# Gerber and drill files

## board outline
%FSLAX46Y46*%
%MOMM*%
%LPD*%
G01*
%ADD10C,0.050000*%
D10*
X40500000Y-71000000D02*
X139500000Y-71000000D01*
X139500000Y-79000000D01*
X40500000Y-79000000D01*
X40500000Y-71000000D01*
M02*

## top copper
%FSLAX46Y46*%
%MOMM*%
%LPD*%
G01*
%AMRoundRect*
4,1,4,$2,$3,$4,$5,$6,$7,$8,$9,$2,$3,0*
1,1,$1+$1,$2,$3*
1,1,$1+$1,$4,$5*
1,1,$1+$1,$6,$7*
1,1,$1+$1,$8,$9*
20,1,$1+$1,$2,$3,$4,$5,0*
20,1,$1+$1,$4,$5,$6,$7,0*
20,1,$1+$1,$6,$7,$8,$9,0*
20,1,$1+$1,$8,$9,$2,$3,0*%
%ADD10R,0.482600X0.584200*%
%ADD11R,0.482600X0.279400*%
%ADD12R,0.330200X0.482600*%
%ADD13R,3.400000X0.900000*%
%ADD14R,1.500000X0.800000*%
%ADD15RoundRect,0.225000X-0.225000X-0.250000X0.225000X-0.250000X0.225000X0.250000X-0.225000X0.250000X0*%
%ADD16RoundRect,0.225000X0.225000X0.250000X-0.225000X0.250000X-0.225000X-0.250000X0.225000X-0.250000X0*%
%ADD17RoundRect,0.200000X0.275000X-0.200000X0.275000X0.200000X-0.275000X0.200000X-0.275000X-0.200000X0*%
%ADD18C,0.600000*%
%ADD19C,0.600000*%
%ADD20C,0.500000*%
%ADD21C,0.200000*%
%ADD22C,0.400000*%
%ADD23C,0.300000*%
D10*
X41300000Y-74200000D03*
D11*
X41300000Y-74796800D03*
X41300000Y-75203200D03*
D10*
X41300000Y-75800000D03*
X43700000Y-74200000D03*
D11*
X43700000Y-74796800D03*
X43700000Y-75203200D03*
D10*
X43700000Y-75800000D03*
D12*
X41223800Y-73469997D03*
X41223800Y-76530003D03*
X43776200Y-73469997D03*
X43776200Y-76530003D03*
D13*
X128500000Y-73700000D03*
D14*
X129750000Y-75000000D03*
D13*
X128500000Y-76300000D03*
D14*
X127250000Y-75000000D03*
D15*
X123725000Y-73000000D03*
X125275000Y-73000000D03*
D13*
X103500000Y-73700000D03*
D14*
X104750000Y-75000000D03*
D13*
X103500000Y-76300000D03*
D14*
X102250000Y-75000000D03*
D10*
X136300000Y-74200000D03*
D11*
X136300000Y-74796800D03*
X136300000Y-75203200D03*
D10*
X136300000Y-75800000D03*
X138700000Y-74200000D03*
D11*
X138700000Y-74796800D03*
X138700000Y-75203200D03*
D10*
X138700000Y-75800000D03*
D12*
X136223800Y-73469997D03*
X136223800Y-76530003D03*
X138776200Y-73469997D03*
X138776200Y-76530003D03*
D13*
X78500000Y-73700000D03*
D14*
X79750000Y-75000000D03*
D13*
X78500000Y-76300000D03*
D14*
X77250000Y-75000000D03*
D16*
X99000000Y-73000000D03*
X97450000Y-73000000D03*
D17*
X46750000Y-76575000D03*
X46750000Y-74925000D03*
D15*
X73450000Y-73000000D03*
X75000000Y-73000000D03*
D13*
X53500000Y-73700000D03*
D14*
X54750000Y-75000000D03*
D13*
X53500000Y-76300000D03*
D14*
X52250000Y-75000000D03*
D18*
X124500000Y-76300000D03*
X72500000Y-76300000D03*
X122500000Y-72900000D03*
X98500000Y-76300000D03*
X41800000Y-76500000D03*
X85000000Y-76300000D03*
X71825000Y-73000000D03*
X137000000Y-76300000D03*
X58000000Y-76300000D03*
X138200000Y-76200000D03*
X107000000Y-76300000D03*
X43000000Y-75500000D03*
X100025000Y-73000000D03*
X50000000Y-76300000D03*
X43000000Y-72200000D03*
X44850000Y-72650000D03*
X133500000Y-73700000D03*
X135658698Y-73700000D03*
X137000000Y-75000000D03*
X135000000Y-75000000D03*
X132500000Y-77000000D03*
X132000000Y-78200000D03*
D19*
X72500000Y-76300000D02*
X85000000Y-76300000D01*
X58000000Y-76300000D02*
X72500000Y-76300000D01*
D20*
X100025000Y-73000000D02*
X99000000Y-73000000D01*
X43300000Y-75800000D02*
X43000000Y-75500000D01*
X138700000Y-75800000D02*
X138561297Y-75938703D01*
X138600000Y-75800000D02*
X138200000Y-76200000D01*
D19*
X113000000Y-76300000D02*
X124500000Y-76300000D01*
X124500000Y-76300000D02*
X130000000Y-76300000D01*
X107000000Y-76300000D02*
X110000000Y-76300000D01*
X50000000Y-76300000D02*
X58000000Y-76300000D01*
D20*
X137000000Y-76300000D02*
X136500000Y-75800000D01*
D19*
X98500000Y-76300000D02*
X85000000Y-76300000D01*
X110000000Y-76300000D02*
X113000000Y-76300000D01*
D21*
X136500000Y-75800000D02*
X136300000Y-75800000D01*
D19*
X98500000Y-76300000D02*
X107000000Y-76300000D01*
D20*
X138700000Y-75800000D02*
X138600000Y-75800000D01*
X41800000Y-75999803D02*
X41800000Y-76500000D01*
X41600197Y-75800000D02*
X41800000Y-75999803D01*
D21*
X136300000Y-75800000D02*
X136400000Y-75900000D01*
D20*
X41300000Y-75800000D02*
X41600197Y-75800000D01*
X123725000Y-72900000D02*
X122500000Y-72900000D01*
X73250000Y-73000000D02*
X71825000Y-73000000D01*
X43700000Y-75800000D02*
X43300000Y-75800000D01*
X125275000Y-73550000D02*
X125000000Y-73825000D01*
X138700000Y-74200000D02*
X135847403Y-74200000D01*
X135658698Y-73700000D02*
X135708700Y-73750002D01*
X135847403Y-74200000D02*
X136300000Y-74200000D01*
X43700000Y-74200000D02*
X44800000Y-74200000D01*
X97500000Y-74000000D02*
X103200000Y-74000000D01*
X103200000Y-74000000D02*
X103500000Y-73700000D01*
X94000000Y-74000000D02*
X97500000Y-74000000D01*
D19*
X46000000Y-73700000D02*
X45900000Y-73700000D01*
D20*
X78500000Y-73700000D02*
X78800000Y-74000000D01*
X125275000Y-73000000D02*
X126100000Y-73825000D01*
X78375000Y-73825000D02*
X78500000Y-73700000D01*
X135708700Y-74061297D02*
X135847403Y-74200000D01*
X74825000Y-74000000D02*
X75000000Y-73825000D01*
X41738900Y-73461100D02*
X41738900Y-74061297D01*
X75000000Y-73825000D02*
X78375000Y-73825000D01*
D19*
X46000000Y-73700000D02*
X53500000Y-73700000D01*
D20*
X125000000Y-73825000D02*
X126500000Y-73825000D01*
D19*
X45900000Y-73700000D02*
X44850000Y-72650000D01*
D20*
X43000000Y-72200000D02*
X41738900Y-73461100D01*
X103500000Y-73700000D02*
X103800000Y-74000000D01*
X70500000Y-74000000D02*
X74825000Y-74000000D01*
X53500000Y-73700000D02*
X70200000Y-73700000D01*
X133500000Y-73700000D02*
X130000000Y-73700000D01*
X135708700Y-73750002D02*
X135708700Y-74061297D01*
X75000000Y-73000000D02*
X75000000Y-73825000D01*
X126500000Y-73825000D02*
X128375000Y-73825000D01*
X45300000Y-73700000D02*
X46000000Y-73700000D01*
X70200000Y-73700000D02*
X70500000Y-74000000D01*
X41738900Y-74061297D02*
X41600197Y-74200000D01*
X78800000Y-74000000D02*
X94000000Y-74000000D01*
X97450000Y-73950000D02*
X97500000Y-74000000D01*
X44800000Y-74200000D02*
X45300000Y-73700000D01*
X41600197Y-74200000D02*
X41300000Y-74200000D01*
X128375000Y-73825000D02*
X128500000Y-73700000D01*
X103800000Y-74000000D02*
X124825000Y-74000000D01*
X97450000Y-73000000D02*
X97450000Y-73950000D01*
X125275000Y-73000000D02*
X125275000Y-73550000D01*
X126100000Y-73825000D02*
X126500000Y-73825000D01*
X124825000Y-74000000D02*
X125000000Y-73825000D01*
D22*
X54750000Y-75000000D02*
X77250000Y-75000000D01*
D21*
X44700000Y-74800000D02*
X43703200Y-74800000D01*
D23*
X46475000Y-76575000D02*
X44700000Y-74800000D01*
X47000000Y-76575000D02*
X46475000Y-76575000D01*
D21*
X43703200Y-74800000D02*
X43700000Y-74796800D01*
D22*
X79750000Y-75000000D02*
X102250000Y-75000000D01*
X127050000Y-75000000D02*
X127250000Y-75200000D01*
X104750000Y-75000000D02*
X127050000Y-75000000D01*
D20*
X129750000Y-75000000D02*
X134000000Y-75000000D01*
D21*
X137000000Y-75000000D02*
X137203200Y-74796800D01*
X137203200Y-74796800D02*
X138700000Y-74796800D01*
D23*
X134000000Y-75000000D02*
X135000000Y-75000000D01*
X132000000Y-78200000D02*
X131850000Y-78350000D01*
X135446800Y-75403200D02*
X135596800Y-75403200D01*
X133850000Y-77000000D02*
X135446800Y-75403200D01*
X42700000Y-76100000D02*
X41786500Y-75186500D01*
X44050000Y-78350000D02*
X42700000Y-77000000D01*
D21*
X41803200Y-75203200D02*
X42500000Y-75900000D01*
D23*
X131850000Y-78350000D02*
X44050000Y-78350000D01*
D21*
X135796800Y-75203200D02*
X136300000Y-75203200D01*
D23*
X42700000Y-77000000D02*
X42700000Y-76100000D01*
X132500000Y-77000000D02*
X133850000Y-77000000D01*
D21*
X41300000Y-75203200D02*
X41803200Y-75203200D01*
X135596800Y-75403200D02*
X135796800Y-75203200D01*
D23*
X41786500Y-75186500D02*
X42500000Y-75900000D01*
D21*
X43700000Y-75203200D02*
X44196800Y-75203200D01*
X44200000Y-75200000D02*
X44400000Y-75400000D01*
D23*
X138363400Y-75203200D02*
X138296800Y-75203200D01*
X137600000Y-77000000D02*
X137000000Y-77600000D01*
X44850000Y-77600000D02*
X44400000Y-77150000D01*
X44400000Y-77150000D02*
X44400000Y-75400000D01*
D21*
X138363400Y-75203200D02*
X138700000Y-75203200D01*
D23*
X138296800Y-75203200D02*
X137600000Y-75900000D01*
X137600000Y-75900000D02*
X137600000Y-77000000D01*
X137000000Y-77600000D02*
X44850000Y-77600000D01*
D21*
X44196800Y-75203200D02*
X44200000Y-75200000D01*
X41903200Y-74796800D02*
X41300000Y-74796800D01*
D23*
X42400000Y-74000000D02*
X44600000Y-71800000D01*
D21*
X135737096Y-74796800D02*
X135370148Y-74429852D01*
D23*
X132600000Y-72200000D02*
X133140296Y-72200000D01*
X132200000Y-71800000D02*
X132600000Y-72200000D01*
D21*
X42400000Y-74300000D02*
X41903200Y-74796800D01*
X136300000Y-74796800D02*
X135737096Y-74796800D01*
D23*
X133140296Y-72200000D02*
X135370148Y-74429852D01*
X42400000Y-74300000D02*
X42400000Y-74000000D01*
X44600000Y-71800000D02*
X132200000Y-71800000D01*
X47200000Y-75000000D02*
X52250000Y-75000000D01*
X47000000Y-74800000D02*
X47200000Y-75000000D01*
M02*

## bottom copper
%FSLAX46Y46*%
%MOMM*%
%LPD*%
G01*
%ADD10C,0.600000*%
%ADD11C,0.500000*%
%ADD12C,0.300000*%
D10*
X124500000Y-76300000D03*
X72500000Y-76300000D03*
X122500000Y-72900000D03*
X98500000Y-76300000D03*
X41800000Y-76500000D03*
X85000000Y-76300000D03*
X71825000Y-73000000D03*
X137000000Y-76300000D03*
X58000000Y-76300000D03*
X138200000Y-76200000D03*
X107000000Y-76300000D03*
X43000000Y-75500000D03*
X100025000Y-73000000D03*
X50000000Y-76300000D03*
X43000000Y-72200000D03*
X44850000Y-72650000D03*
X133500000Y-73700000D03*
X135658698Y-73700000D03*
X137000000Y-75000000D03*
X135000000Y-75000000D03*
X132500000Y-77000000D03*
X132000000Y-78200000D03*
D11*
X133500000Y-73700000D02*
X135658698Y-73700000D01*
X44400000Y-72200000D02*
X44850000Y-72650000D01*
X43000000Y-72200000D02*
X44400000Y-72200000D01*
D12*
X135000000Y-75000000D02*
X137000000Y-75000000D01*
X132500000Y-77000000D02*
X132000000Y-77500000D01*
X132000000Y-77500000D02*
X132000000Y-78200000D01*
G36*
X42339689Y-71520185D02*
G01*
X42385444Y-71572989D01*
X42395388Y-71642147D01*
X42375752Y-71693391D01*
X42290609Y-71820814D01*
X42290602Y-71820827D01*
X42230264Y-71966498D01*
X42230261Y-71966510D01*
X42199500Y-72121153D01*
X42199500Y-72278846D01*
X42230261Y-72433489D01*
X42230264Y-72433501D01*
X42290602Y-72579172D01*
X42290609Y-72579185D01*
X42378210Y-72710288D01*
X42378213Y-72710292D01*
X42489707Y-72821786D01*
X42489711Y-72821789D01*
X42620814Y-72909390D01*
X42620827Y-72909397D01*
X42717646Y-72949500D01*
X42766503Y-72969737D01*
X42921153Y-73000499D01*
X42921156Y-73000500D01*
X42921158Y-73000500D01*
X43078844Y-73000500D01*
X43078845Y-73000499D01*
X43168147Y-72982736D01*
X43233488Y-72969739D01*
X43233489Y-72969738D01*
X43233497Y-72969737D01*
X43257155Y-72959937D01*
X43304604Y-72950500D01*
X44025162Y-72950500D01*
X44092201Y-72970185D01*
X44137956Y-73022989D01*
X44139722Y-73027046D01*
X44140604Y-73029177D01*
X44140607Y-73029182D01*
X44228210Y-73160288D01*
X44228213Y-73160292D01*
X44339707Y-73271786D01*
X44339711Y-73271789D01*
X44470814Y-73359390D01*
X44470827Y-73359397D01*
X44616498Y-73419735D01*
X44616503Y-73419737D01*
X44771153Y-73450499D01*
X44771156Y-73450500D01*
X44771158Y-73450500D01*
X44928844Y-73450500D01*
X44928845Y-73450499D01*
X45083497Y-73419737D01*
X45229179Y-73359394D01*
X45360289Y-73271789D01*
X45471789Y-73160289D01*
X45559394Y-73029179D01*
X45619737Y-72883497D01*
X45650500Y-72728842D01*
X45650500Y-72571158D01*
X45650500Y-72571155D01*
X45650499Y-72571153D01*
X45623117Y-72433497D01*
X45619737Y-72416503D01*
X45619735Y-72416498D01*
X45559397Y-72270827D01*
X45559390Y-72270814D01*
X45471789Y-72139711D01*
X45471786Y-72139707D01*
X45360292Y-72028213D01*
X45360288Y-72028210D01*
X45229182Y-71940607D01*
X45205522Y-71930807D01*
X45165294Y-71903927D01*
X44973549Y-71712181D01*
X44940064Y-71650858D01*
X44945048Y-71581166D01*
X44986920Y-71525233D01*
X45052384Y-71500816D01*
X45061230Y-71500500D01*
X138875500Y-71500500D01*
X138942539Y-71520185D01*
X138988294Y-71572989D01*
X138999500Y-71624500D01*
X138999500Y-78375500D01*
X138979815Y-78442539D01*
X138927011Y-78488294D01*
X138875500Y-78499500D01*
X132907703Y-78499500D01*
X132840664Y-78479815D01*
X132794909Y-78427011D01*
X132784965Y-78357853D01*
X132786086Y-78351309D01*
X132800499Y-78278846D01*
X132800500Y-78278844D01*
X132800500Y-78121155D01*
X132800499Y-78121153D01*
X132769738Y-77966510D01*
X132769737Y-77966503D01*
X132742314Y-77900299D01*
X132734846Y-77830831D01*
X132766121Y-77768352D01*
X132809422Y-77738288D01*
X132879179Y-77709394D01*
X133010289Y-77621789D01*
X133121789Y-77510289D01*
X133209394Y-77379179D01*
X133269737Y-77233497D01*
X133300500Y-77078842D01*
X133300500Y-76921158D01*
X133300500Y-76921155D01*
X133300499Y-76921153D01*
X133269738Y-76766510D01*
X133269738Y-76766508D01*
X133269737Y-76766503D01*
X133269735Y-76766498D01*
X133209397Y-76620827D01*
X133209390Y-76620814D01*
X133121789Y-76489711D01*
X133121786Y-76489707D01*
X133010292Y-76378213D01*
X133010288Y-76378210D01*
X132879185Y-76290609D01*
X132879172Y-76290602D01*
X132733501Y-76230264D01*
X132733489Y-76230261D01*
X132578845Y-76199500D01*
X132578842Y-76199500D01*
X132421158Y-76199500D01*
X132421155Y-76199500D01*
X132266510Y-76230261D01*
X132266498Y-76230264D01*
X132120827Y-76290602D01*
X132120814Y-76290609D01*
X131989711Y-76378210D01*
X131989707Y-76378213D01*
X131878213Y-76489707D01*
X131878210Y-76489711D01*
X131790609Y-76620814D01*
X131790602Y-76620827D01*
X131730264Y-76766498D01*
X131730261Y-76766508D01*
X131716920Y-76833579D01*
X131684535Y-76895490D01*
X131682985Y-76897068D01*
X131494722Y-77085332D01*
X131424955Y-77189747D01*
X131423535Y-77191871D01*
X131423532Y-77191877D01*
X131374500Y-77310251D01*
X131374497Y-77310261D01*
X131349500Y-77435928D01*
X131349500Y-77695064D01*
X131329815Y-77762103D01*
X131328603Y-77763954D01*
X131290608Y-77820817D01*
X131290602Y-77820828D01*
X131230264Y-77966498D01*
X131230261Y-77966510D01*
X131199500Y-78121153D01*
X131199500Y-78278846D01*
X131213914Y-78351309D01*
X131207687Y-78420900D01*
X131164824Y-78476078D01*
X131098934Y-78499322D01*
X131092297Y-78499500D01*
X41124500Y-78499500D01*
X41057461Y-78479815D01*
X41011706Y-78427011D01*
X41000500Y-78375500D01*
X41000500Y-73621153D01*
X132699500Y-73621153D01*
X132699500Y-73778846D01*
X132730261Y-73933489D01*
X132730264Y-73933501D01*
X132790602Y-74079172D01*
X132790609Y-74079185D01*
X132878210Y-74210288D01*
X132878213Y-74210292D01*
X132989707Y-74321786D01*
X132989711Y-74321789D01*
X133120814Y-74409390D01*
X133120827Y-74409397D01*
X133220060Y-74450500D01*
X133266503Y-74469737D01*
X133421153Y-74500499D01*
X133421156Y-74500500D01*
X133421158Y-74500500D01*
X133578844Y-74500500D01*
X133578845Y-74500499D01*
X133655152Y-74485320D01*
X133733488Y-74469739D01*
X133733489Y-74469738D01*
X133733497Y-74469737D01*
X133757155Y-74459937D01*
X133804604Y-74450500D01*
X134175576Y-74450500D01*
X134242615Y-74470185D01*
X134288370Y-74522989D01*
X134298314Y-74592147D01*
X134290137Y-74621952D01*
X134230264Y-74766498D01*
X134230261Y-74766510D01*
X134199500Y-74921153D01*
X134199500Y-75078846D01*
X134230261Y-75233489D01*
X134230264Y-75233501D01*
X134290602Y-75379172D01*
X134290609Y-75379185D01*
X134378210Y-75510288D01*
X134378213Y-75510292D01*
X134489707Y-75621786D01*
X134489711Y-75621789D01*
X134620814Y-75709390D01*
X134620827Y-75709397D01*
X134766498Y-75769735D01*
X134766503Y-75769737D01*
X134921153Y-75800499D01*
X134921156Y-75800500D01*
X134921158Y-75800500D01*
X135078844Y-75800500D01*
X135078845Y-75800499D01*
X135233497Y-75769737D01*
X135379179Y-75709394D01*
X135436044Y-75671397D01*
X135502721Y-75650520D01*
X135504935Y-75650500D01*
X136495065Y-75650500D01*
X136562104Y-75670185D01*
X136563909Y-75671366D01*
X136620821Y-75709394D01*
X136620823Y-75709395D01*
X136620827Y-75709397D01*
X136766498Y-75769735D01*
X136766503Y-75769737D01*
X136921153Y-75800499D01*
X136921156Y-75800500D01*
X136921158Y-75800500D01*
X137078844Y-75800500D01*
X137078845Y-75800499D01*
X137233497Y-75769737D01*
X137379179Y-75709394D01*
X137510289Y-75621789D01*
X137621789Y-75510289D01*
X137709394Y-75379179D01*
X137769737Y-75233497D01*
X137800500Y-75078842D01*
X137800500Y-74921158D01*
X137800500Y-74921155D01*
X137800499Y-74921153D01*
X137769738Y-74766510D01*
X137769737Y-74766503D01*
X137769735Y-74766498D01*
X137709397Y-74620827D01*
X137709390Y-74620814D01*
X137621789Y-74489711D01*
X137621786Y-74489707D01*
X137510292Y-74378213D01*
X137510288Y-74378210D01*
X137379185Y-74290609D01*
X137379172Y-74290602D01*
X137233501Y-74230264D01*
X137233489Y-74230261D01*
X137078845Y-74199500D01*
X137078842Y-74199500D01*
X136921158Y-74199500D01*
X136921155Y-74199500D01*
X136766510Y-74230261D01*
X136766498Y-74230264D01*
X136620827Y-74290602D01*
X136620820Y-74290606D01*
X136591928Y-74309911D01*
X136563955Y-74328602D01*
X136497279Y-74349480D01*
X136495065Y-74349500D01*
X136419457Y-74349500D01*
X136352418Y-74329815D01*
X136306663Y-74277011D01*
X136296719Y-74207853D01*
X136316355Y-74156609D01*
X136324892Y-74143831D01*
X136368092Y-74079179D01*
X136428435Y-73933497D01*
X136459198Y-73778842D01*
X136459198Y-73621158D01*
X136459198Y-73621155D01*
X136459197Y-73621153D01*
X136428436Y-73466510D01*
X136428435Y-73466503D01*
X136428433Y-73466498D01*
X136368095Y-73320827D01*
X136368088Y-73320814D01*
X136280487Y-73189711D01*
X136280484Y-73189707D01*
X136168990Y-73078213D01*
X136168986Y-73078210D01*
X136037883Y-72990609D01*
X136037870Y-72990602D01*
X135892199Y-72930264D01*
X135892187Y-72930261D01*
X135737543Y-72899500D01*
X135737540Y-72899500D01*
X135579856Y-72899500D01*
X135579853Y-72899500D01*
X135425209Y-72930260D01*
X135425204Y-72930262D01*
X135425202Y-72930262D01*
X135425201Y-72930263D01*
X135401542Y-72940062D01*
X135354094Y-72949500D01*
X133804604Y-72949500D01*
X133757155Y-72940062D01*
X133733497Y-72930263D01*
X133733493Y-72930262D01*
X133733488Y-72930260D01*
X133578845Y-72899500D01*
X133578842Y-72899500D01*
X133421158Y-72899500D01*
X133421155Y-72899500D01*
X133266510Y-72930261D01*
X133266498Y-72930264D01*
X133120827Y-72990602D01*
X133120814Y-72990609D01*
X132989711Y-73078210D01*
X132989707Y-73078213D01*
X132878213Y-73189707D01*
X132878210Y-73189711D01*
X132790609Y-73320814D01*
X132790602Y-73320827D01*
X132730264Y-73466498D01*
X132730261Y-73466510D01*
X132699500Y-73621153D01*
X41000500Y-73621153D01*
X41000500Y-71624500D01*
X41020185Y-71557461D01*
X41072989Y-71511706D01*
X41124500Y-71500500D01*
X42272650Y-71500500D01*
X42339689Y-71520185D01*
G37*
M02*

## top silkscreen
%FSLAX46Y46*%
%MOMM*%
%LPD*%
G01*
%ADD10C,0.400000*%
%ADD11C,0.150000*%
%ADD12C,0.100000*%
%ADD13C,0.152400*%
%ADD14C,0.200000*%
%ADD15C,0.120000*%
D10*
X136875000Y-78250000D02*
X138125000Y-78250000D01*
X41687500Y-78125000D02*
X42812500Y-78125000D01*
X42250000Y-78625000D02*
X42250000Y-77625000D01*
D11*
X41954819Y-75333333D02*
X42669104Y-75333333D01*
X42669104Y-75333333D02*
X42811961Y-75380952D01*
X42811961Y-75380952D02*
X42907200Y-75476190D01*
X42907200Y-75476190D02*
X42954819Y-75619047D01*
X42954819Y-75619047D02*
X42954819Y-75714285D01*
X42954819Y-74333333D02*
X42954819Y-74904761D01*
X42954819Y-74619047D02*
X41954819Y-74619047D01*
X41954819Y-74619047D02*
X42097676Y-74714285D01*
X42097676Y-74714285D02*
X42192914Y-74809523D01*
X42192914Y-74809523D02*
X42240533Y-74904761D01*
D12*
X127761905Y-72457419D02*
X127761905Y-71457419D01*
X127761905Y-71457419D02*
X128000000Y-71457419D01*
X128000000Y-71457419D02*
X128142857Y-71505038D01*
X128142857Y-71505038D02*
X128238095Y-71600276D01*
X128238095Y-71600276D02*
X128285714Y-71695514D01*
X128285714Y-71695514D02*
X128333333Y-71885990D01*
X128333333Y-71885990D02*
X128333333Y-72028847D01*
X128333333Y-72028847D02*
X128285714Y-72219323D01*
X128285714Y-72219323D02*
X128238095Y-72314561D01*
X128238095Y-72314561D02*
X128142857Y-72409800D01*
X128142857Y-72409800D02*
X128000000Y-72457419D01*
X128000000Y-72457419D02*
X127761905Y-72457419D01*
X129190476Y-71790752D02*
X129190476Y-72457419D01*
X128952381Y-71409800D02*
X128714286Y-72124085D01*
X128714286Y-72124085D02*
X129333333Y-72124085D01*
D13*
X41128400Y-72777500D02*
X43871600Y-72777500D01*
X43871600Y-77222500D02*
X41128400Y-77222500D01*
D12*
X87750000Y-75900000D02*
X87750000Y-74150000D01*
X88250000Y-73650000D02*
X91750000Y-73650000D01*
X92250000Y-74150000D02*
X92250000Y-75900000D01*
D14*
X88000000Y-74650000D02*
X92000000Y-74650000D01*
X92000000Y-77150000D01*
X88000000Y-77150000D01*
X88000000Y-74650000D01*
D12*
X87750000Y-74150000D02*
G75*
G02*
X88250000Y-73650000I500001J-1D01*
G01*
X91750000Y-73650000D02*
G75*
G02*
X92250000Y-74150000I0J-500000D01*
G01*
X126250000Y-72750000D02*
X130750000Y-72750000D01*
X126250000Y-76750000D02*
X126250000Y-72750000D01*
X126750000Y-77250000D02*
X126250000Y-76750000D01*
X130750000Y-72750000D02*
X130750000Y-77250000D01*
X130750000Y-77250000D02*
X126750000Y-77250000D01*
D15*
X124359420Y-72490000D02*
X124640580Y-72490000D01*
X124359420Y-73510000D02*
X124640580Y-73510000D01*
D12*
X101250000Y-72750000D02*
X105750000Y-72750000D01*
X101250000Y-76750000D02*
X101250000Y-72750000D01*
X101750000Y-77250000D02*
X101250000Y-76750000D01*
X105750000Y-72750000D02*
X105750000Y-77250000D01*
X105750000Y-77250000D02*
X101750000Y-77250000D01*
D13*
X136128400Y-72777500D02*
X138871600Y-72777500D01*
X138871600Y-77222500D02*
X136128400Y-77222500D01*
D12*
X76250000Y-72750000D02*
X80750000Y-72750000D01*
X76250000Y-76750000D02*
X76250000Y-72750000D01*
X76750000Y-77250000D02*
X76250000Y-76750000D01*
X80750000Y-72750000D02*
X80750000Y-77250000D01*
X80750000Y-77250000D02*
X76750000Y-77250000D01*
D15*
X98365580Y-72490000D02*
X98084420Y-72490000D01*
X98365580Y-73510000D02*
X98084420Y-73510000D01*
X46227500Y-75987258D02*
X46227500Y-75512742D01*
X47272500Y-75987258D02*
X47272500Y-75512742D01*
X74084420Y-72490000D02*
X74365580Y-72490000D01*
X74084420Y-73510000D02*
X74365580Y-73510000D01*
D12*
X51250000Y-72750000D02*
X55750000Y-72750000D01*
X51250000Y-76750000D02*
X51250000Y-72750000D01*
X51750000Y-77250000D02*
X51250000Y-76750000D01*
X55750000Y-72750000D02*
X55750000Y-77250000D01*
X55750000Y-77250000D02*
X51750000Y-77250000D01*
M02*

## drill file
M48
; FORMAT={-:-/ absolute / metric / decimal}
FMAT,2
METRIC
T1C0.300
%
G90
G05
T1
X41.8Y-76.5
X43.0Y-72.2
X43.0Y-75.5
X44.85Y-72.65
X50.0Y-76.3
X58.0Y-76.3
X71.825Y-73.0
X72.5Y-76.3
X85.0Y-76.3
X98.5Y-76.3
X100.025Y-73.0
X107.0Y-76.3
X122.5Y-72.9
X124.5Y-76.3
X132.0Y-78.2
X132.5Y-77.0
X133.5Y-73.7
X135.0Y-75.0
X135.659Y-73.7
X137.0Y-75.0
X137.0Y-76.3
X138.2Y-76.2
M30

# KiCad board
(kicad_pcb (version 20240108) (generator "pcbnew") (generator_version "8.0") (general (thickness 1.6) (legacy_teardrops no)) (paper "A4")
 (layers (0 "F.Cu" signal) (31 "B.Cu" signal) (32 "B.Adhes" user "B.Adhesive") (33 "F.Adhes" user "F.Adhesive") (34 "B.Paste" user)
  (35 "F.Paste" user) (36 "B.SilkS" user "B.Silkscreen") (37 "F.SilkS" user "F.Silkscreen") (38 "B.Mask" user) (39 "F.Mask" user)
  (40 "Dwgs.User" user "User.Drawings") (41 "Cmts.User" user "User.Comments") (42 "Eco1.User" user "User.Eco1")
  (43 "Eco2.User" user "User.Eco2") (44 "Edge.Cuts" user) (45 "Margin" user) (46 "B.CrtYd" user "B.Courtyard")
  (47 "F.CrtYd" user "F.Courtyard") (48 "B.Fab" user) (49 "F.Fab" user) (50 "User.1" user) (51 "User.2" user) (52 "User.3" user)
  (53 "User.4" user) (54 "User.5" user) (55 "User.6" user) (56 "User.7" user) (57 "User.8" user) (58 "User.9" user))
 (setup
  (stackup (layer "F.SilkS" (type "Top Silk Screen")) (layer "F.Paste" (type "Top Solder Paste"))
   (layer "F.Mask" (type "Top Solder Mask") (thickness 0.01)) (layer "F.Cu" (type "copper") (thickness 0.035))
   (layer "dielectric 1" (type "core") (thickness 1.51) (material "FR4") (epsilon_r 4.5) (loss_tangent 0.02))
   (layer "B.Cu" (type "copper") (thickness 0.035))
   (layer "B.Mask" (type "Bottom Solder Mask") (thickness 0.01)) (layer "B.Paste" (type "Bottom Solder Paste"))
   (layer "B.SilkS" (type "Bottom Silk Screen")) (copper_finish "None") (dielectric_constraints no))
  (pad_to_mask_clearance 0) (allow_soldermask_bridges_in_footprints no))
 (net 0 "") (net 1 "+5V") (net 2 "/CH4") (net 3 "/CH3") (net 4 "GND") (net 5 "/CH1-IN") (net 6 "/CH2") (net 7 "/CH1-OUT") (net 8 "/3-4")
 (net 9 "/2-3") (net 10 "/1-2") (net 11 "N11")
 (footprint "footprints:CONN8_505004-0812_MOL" (layer "F.Cu") (at 42.5 75 90)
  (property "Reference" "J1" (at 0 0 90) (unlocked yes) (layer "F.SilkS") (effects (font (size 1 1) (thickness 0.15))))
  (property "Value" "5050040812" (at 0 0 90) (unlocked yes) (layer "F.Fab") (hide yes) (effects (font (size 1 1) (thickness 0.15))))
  (fp_line (start 2.2225 -1.3716) (end 2.2225 1.3716) (stroke (width 0.1524) (type solid)) (layer "F.SilkS"))
  (fp_line (start -2.2225 1.3716) (end -2.2225 -1.3716) (stroke (width 0.1524) (type solid)) (layer "F.SilkS"))
  (pad "1" smd rect (at 0.8 -1.2 90) (size 0.5842 0.4826) (layers "F.Cu" "F.Paste" "F.Mask") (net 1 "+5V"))
  (pad "2" smd rect (at 0.2032 -1.2 90) (size 0.2794 0.4826) (layers "F.Cu" "F.Paste" "F.Mask") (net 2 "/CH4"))
  (pad "3" smd rect (at -0.2032 -1.2 90) (size 0.2794 0.4826) (layers "F.Cu" "F.Paste" "F.Mask") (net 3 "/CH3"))
  (pad "4" smd rect (at -0.8 -1.2 90) (size 0.5842 0.4826) (layers "F.Cu" "F.Paste" "F.Mask") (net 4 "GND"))
  (pad "5" smd rect (at 0.8 1.2 90) (size 0.5842 0.4826) (layers "F.Cu" "F.Paste" "F.Mask") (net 1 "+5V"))
  (pad "6" smd rect (at 0.2032 1.2 90) (size 0.2794 0.4826) (layers "F.Cu" "F.Paste" "F.Mask") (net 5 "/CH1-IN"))
  (pad "7" smd rect (at -0.2032 1.2 90) (size 0.2794 0.4826) (layers "F.Cu" "F.Paste" "F.Mask") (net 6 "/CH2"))
  (pad "8" smd rect (at -0.8 1.2 90) (size 0.5842 0.4826) (layers "F.Cu" "F.Paste" "F.Mask") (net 4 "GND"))
  (pad "9" smd rect (at 1.530003 -1.2762 90) (size 0.4826 0.3302) (layers "F.Cu" "F.Paste" "F.Mask"))
  (pad "10" smd rect (at -1.530003 -1.2762 90) (size 0.4826 0.3302) (layers "F.Cu" "F.Paste" "F.Mask"))
  (pad "11" smd rect (at 1.530003 1.2762 90) (size 0.4826 0.3302) (layers "F.Cu" "F.Paste" "F.Mask"))
  (pad "12" smd rect (at -1.530003 1.2762 90) (size 0.4826 0.3302) (layers "F.Cu" "F.Paste" "F.Mask")))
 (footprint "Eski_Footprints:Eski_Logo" (layer "F.Cu") (at 90 77.15)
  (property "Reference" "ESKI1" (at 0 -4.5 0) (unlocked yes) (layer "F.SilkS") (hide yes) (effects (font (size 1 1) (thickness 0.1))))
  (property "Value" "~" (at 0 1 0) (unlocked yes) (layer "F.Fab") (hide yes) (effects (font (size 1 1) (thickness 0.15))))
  (fp_line (start -2.25 -1.25) (end -2.25 -3) (stroke (width 0.1) (type default)) (layer "F.SilkS"))
  (fp_line (start -1.75 -3.5) (end 1.75 -3.5) (stroke (width 0.1) (type default)) (layer "F.SilkS"))
  (fp_line (start 2.25 -3) (end 2.25 -1.25) (stroke (width 0.1) (type default)) (layer "F.SilkS"))
  (fp_rect (start -2 -2.5) (end 2 0) (stroke (width 0.2) (type default)) (fill none) (layer "F.SilkS"))
  (fp_arc (start -2.25 -3) (mid -2.103553 -3.353553) (end -1.75 -3.5) (stroke (width 0.1) (type default)) (layer "F.SilkS"))
  (fp_arc (start 1.75 -3.5) (mid 2.103553 -3.353553) (end 2.25 -3) (stroke (width 0.1) (type default)) (layer "F.SilkS")))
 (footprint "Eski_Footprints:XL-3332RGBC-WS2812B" (layer "F.Cu") (at 128.5 75)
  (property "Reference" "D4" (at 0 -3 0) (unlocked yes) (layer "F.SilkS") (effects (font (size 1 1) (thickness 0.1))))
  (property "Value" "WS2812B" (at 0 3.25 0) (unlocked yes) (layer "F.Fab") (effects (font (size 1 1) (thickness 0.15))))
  (fp_line (start -2.25 -2.25) (end 2.25 -2.25) (stroke (width 0.1) (type default)) (layer "F.SilkS"))
  (fp_line (start -2.25 1.75) (end -2.25 -2.25) (stroke (width 0.1) (type default)) (layer "F.SilkS"))
  (fp_line (start -1.75 2.25) (end -2.25 1.75) (stroke (width 0.1) (type default)) (layer "F.SilkS"))
  (fp_line (start 2.25 -2.25) (end 2.25 2.25) (stroke (width 0.1) (type default)) (layer "F.SilkS"))
  (fp_line (start 2.25 2.25) (end -1.75 2.25) (stroke (width 0.1) (type default)) (layer "F.SilkS"))
  (pad "1" smd rect (at 0 -1.3) (size 3.4 0.9) (layers "F.Cu" "F.Paste" "F.Mask") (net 1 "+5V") (thermal_bridge_angle 45))
  (pad "2" smd rect (at 1.25 0) (size 1.5 0.8) (layers "F.Cu" "F.Paste" "F.Mask") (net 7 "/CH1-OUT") (thermal_bridge_angle 45))
  (pad "3" smd rect (at 0 1.3) (size 3.4 0.9) (layers "F.Cu" "F.Paste" "F.Mask") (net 4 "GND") (thermal_bridge_angle 45))
  (pad "4" smd rect (at -1.25 0) (size 1.5 0.8) (layers "F.Cu" "F.Paste" "F.Mask") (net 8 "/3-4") (thermal_bridge_angle 45)))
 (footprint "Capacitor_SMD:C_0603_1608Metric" (layer "F.Cu") (at 124.5 73)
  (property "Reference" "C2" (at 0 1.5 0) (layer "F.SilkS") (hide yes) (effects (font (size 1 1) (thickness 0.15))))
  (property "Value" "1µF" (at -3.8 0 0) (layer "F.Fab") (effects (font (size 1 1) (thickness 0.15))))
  (fp_line (start -0.14058 -0.51) (end 0.14058 -0.51) (stroke (width 0.12) (type solid)) (layer "F.SilkS"))
  (fp_line (start -0.14058 0.51) (end 0.14058 0.51) (stroke (width 0.12) (type solid)) (layer "F.SilkS"))
  (pad "1" smd roundrect (at -0.775 0) (size 0.9 0.95) (layers "F.Cu" "F.Paste" "F.Mask") (roundrect_rratio 0.25) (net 4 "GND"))
  (pad "2" smd roundrect (at 0.775 0) (size 0.9 0.95) (layers "F.Cu" "F.Paste" "F.Mask") (roundrect_rratio 0.25) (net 1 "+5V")))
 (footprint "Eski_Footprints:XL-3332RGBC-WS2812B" (layer "F.Cu") (at 103.5 75)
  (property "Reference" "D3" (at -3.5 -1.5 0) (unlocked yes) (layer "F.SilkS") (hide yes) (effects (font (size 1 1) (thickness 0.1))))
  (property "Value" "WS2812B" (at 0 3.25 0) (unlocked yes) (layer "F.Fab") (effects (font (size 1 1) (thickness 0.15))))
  (fp_line (start -2.25 -2.25) (end 2.25 -2.25) (stroke (width 0.1) (type default)) (layer "F.SilkS"))
  (fp_line (start -2.25 1.75) (end -2.25 -2.25) (stroke (width 0.1) (type default)) (layer "F.SilkS"))
  (fp_line (start -1.75 2.25) (end -2.25 1.75) (stroke (width 0.1) (type default)) (layer "F.SilkS"))
  (fp_line (start 2.25 -2.25) (end 2.25 2.25) (stroke (width 0.1) (type default)) (layer "F.SilkS"))
  (fp_line (start 2.25 2.25) (end -1.75 2.25) (stroke (width 0.1) (type default)) (layer "F.SilkS"))
  (pad "1" smd rect (at 0 -1.3) (size 3.4 0.9) (layers "F.Cu" "F.Paste" "F.Mask") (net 1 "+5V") (thermal_bridge_angle 45))
  (pad "2" smd rect (at 1.25 0) (size 1.5 0.8) (layers "F.Cu" "F.Paste" "F.Mask") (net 8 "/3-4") (thermal_bridge_angle 45))
  (pad "3" smd rect (at 0 1.3) (size 3.4 0.9) (layers "F.Cu" "F.Paste" "F.Mask") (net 4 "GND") (thermal_bridge_angle 45))
  (pad "4" smd rect (at -1.25 0) (size 1.5 0.8) (layers "F.Cu" "F.Paste" "F.Mask") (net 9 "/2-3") (thermal_bridge_angle 45)))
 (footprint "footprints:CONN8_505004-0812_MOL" (layer "F.Cu") (at 137.5 75 90)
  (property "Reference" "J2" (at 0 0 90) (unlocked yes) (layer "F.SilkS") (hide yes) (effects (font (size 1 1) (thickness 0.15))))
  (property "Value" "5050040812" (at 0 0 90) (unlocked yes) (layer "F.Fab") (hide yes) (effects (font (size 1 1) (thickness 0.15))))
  (fp_line (start 2.2225 -1.3716) (end 2.2225 1.3716) (stroke (width 0.1524) (type solid)) (layer "F.SilkS"))
  (fp_line (start -2.2225 1.3716) (end -2.2225 -1.3716) (stroke (width 0.1524) (type solid)) (layer "F.SilkS"))
  (pad "1" smd rect (at 0.8 -1.2 90) (size 0.5842 0.4826) (layers "F.Cu" "F.Paste" "F.Mask") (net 1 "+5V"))
  (pad "2" smd rect (at 0.2032 -1.2 90) (size 0.2794 0.4826) (layers "F.Cu" "F.Paste" "F.Mask") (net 2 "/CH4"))
  (pad "3" smd rect (at -0.2032 -1.2 90) (size 0.2794 0.4826) (layers "F.Cu" "F.Paste" "F.Mask") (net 3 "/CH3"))
  (pad "4" smd rect (at -0.8 -1.2 90) (size 0.5842 0.4826) (layers "F.Cu" "F.Paste" "F.Mask") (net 4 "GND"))
  (pad "5" smd rect (at 0.8 1.2 90) (size 0.5842 0.4826) (layers "F.Cu" "F.Paste" "F.Mask") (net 1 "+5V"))
  (pad "6" smd rect (at 0.2032 1.2 90) (size 0.2794 0.4826) (layers "F.Cu" "F.Paste" "F.Mask") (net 7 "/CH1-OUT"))
  (pad "7" smd rect (at -0.2032 1.2 90) (size 0.2794 0.4826) (layers "F.Cu" "F.Paste" "F.Mask") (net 6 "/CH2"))
  (pad "8" smd rect (at -0.8 1.2 90) (size 0.5842 0.4826) (layers "F.Cu" "F.Paste" "F.Mask") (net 4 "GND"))
  (pad "9" smd rect (at 1.530003 -1.2762 90) (size 0.4826 0.3302) (layers "F.Cu" "F.Paste" "F.Mask"))
  (pad "10" smd rect (at -1.530003 -1.2762 90) (size 0.4826 0.3302) (layers "F.Cu" "F.Paste" "F.Mask"))
  (pad "11" smd rect (at 1.530003 1.2762 90) (size 0.4826 0.3302) (layers "F.Cu" "F.Paste" "F.Mask"))
  (pad "12" smd rect (at -1.530003 1.2762 90) (size 0.4826 0.3302) (layers "F.Cu" "F.Paste" "F.Mask")))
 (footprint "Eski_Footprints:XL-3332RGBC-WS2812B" (layer "F.Cu") (at 78.5 75)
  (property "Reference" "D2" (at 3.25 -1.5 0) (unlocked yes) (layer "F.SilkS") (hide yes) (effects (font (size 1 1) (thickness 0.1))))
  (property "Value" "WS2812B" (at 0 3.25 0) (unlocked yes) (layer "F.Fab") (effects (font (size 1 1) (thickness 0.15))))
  (fp_line (start -2.25 -2.25) (end 2.25 -2.25) (stroke (width 0.1) (type default)) (layer "F.SilkS"))
  (fp_line (start -2.25 1.75) (end -2.25 -2.25) (stroke (width 0.1) (type default)) (layer "F.SilkS"))
  (fp_line (start -1.75 2.25) (end -2.25 1.75) (stroke (width 0.1) (type default)) (layer "F.SilkS"))
  (fp_line (start 2.25 -2.25) (end 2.25 2.25) (stroke (width 0.1) (type default)) (layer "F.SilkS"))
  (fp_line (start 2.25 2.25) (end -1.75 2.25) (stroke (width 0.1) (type default)) (layer "F.SilkS"))
  (pad "1" smd rect (at 0 -1.3) (size 3.4 0.9) (layers "F.Cu" "F.Paste" "F.Mask") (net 1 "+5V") (thermal_bridge_angle 45))
  (pad "2" smd rect (at 1.25 0) (size 1.5 0.8) (layers "F.Cu" "F.Paste" "F.Mask") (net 9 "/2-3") (thermal_bridge_angle 45))
  (pad "3" smd rect (at 0 1.3) (size 3.4 0.9) (layers "F.Cu" "F.Paste" "F.Mask") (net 4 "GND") (thermal_bridge_angle 45))
  (pad "4" smd rect (at -1.25 0) (size 1.5 0.8) (layers "F.Cu" "F.Paste" "F.Mask") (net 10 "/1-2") (thermal_bridge_angle 45)))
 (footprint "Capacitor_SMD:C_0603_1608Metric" (layer "F.Cu") (at 98.225 73 180)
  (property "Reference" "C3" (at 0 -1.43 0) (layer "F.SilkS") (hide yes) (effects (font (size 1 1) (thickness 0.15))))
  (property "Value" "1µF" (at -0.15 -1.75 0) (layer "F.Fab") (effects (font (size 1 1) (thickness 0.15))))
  (fp_line (start -0.14058 0.51) (end 0.14058 0.51) (stroke (width 0.12) (type solid)) (layer "F.SilkS"))
  (fp_line (start -0.14058 -0.51) (end 0.14058 -0.51) (stroke (width 0.12) (type solid)) (layer "F.SilkS"))
  (pad "1" smd roundrect (at -0.775 0 180) (size 0.9 0.95) (layers "F.Cu" "F.Paste" "F.Mask") (roundrect_rratio 0.25) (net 4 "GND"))
  (pad "2" smd roundrect (at 0.775 0 180) (size 0.9 0.95) (layers "F.Cu" "F.Paste" "F.Mask") (roundrect_rratio 0.25) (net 1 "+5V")))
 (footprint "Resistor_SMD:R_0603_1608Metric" (layer "F.Cu") (at 46.75 75.75 90)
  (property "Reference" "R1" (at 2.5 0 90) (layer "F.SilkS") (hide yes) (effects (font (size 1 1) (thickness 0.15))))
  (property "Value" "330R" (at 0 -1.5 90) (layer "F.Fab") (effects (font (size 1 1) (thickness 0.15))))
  (fp_line (start -0.237258 -0.5225) (end 0.237258 -0.5225) (stroke (width 0.12) (type solid)) (layer "F.SilkS"))
  (fp_line (start -0.237258 0.5225) (end 0.237258 0.5225) (stroke (width 0.12) (type solid)) (layer "F.SilkS"))
  (pad "1" smd roundrect (at -0.825 0 90) (size 0.8 0.95) (layers "F.Cu" "F.Paste" "F.Mask") (roundrect_rratio 0.25) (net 5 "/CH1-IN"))
  (pad "2" smd roundrect (at 0.825 0 90) (size 0.8 0.95) (layers "F.Cu" "F.Paste" "F.Mask") (roundrect_rratio 0.25) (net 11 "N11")))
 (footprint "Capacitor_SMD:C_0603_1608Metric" (layer "F.Cu") (at 74.225 73)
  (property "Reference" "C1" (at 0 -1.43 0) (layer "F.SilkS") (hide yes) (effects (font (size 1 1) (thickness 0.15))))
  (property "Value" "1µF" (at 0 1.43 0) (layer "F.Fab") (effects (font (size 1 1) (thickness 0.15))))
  (fp_line (start -0.14058 -0.51) (end 0.14058 -0.51) (stroke (width 0.12) (type solid)) (layer "F.SilkS"))
  (fp_line (start -0.14058 0.51) (end 0.14058 0.51) (stroke (width 0.12) (type solid)) (layer "F.SilkS"))
  (pad "1" smd roundrect (at -0.775 0) (size 0.9 0.95) (layers "F.Cu" "F.Paste" "F.Mask") (roundrect_rratio 0.25) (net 4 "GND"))
  (pad "2" smd roundrect (at 0.775 0) (size 0.9 0.95) (layers "F.Cu" "F.Paste" "F.Mask") (roundrect_rratio 0.25) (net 1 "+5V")))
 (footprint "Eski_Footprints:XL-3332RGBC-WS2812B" (layer "F.Cu") (at 53.5 75)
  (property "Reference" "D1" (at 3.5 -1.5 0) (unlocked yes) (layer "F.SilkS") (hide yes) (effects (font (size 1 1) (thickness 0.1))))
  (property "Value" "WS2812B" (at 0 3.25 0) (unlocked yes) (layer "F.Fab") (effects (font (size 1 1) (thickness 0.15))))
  (fp_line (start -2.25 -2.25) (end 2.25 -2.25) (stroke (width 0.1) (type default)) (layer "F.SilkS"))
  (fp_line (start -2.25 1.75) (end -2.25 -2.25) (stroke (width 0.1) (type default)) (layer "F.SilkS"))
  (fp_line (start -1.75 2.25) (end -2.25 1.75) (stroke (width 0.1) (type default)) (layer "F.SilkS"))
  (fp_line (start 2.25 -2.25) (end 2.25 2.25) (stroke (width 0.1) (type default)) (layer "F.SilkS"))
  (fp_line (start 2.25 2.25) (end -1.75 2.25) (stroke (width 0.1) (type default)) (layer "F.SilkS"))
  (pad "1" smd rect (at 0 -1.3) (size 3.4 0.9) (layers "F.Cu" "F.Paste" "F.Mask") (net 1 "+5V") (thermal_bridge_angle 45))
  (pad "2" smd rect (at 1.25 0) (size 1.5 0.8) (layers "F.Cu" "F.Paste" "F.Mask") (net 10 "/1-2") (thermal_bridge_angle 45))
  (pad "3" smd rect (at 0 1.3) (size 3.4 0.9) (layers "F.Cu" "F.Paste" "F.Mask") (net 4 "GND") (thermal_bridge_angle 45))
  (pad "4" smd rect (at -1.25 0) (size 1.5 0.8) (layers "F.Cu" "F.Paste" "F.Mask") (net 11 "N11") (thermal_bridge_angle 45)))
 (gr_line (start 136.875 78.25) (end 138.125 78.25) (stroke (width 0.4) (type default)) (layer "F.SilkS"))
 (gr_line (start 41.6875 78.125) (end 42.8125 78.125) (stroke (width 0.4) (type default)) (layer "F.SilkS"))
 (gr_line (start 42.25 78.625) (end 42.25 77.625) (stroke (width 0.4) (type default)) (layer "F.SilkS"))
 (gr_rect (start 40.5 71) (end 139.5 79) (stroke (width 0.05) (type default)) (fill none) (layer "Edge.Cuts"))
 (segment (start 72.5 76.3) (end 85 76.3) (width 0.6) (layer "F.Cu") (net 4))
 (segment (start 58 76.3) (end 72.5 76.3) (width 0.6) (layer "F.Cu") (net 4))
 (segment (start 100.025 73) (end 99 73) (width 0.5) (layer "F.Cu") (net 4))
 (segment (start 43.3 75.8) (end 43 75.5) (width 0.5) (layer "F.Cu") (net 4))
 (segment (start 138.7 75.8) (end 138.561297 75.938703) (width 0.5) (layer "F.Cu") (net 4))
 (segment (start 138.6 75.8) (end 138.2 76.2) (width 0.5) (layer "F.Cu") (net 4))
 (segment (start 113 76.3) (end 124.5 76.3) (width 0.6) (layer "F.Cu") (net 4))
 (segment (start 124.5 76.3) (end 130 76.3) (width 0.6) (layer "F.Cu") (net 4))
 (segment (start 107 76.3) (end 110 76.3) (width 0.6) (layer "F.Cu") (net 4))
 (segment (start 50 76.3) (end 58 76.3) (width 0.6) (layer "F.Cu") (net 4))
 (segment (start 137 76.3) (end 136.5 75.8) (width 0.5) (layer "F.Cu") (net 4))
 (segment (start 98.5 76.3) (end 85 76.3) (width 0.6) (layer "F.Cu") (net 4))
 (segment (start 110 76.3) (end 113 76.3) (width 0.6) (layer "F.Cu") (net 4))
 (segment (start 136.5 75.8) (end 136.3 75.8) (width 0.2) (layer "F.Cu") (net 4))
 (segment (start 98.5 76.3) (end 107 76.3) (width 0.6) (layer "F.Cu") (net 4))
 (segment (start 138.7 75.8) (end 138.6 75.8) (width 0.5) (layer "F.Cu") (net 4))
 (segment (start 41.8 75.999803) (end 41.8 76.5) (width 0.5) (layer "F.Cu") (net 4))
 (segment (start 41.600197 75.8) (end 41.8 75.999803) (width 0.5) (layer "F.Cu") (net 4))
 (segment (start 136.3 75.8) (end 136.4 75.9) (width 0.2) (layer "F.Cu") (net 4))
 (segment (start 41.3 75.8) (end 41.600197 75.8) (width 0.5) (layer "F.Cu") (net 4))
 (segment (start 123.725 72.9) (end 122.5 72.9) (width 0.5) (layer "F.Cu") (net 4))
 (segment (start 73.25 73) (end 71.825 73) (width 0.5) (layer "F.Cu") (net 4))
 (segment (start 43.7 75.8) (end 43.3 75.8) (width 0.5) (layer "F.Cu") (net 4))
 (via (at 124.5 76.3) (size 0.6) (drill 0.3) (layers "F.Cu" "B.Cu") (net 4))
 (via (at 72.5 76.3) (size 0.6) (drill 0.3) (layers "F.Cu" "B.Cu") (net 4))
 (via (at 122.5 72.9) (size 0.6) (drill 0.3) (layers "F.Cu" "B.Cu") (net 4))
 (via (at 98.5 76.3) (size 0.6) (drill 0.3) (layers "F.Cu" "B.Cu") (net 4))
 (via (at 41.8 76.5) (size 0.6) (drill 0.3) (layers "F.Cu" "B.Cu") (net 4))
 (via (at 85 76.3) (size 0.6) (drill 0.3) (layers "F.Cu" "B.Cu") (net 4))
 (via (at 71.825 73) (size 0.6) (drill 0.3) (layers "F.Cu" "B.Cu") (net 4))
 (via (at 137 76.3) (size 0.6) (drill 0.3) (layers "F.Cu" "B.Cu") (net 4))
 (via (at 58 76.3) (size 0.6) (drill 0.3) (layers "F.Cu" "B.Cu") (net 4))
 (via (at 138.2 76.2) (size 0.6) (drill 0.3) (layers "F.Cu" "B.Cu") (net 4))
 (via (at 107 76.3) (size 0.6) (drill 0.3) (layers "F.Cu" "B.Cu") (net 4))
 (via (at 43 75.5) (size 0.6) (drill 0.3) (layers "F.Cu" "B.Cu") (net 4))
 (via (at 100.025 73) (size 0.6) (drill 0.3) (layers "F.Cu" "B.Cu") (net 4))
 (via (at 50 76.3) (size 0.6) (drill 0.3) (layers "F.Cu" "B.Cu") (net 4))
 (segment (start 125.275 73.55) (end 125 73.825) (width 0.5) (layer "F.Cu") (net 1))
 (segment (start 138.7 74.2) (end 135.847403 74.2) (width 0.5) (layer "F.Cu") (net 1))
 (segment (start 135.658698 73.7) (end 135.7087 73.750002) (width 0.5) (layer "F.Cu") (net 1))
 (segment (start 135.847403 74.2) (end 136.3 74.2) (width 0.5) (layer "F.Cu") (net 1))
 (segment (start 43.7 74.2) (end 44.8 74.2) (width 0.5) (layer "F.Cu") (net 1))
 (segment (start 97.5 74) (end 103.2 74) (width 0.5) (layer "F.Cu") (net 1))
 (segment (start 103.2 74) (end 103.5 73.7) (width 0.5) (layer "F.Cu") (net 1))
 (segment (start 94 74) (end 97.5 74) (width 0.5) (layer "F.Cu") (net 1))
 (segment (start 46 73.7) (end 45.9 73.7) (width 0.6) (layer "F.Cu") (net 1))
 (segment (start 78.5 73.7) (end 78.8 74) (width 0.5) (layer "F.Cu") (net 1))
 (segment (start 125.275 73) (end 126.1 73.825) (width 0.5) (layer "F.Cu") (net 1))
 (segment (start 78.375 73.825) (end 78.5 73.7) (width 0.5) (layer "F.Cu") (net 1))
 (segment (start 135.7087 74.061297) (end 135.847403 74.2) (width 0.5) (layer "F.Cu") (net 1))
 (segment (start 74.825 74) (end 75 73.825) (width 0.5) (layer "F.Cu") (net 1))
 (segment (start 41.7389 73.4611) (end 41.7389 74.061297) (width 0.5) (layer "F.Cu") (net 1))
 (segment (start 75 73.825) (end 78.375 73.825) (width 0.5) (layer "F.Cu") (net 1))
 (segment (start 46 73.7) (end 53.5 73.7) (width 0.6) (layer "F.Cu") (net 1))
 (segment (start 125 73.825) (end 126.5 73.825) (width 0.5) (layer "F.Cu") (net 1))
 (segment (start 45.9 73.7) (end 44.85 72.65) (width 0.6) (layer "F.Cu") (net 1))
 (segment (start 43 72.2) (end 41.7389 73.4611) (width 0.5) (layer "F.Cu") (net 1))
 (segment (start 103.5 73.7) (end 103.8 74) (width 0.5) (layer "F.Cu") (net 1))
 (segment (start 70.5 74) (end 74.825 74) (width 0.5) (layer "F.Cu") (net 1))
 (segment (start 53.5 73.7) (end 70.2 73.7) (width 0.5) (layer "F.Cu") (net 1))
 (segment (start 133.5 73.7) (end 130 73.7) (width 0.5) (layer "F.Cu") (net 1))
 (segment (start 135.7087 73.750002) (end 135.7087 74.061297) (width 0.5) (layer "F.Cu") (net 1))
 (segment (start 75 73) (end 75 73.825) (width 0.5) (layer "F.Cu") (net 1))
 (segment (start 126.5 73.825) (end 128.375 73.825) (width 0.5) (layer "F.Cu") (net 1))
 (segment (start 45.3 73.7) (end 46 73.7) (width 0.5) (layer "F.Cu") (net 1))
 (segment (start 70.2 73.7) (end 70.5 74) (width 0.5) (layer "F.Cu") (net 1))
 (segment (start 41.7389 74.061297) (end 41.600197 74.2) (width 0.5) (layer "F.Cu") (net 1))
 (segment (start 78.8 74) (end 94 74) (width 0.5) (layer "F.Cu") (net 1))
 (segment (start 97.45 73.95) (end 97.5 74) (width 0.5) (layer "F.Cu") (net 1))
 (segment (start 44.8 74.2) (end 45.3 73.7) (width 0.5) (layer "F.Cu") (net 1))
 (segment (start 41.600197 74.2) (end 41.3 74.2) (width 0.5) (layer "F.Cu") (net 1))
 (segment (start 128.375 73.825) (end 128.5 73.7) (width 0.5) (layer "F.Cu") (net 1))
 (segment (start 103.8 74) (end 124.825 74) (width 0.5) (layer "F.Cu") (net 1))
 (segment (start 97.45 73) (end 97.45 73.95) (width 0.5) (layer "F.Cu") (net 1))
 (segment (start 125.275 73) (end 125.275 73.55) (width 0.5) (layer "F.Cu") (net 1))
 (segment (start 126.1 73.825) (end 126.5 73.825) (width 0.5) (layer "F.Cu") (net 1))
 (segment (start 124.825 74) (end 125 73.825) (width 0.5) (layer "F.Cu") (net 1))
 (via (at 43 72.2) (size 0.6) (drill 0.3) (layers "F.Cu" "B.Cu") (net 1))
 (via (at 44.85 72.65) (size 0.6) (drill 0.3) (layers "F.Cu" "B.Cu") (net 1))
 (via (at 133.5 73.7) (size 0.6) (drill 0.3) (layers "F.Cu" "B.Cu") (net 1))
 (via (at 135.658698 73.7) (size 0.6) (drill 0.3) (layers "F.Cu" "B.Cu") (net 1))
 (segment (start 133.5 73.7) (end 135.658698 73.7) (width 0.5) (layer "B.Cu") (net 1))
 (segment (start 44.4 72.2) (end 44.85 72.65) (width 0.5) (layer "B.Cu") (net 1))
 (segment (start 43 72.2) (end 44.4 72.2) (width 0.5) (layer "B.Cu") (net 1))
 (segment (start 54.75 75) (end 77.25 75) (width 0.4) (layer "F.Cu") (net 10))
 (segment (start 44.7 74.8) (end 43.7032 74.8) (width 0.2) (layer "F.Cu") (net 5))
 (segment (start 46.475 76.575) (end 44.7 74.8) (width 0.3) (layer "F.Cu") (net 5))
 (segment (start 47 76.575) (end 46.475 76.575) (width 0.3) (layer "F.Cu") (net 5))
 (segment (start 43.7032 74.8) (end 43.7 74.7968) (width 0.2) (layer "F.Cu") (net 5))
 (segment (start 79.75 75) (end 102.25 75) (width 0.4) (layer "F.Cu") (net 9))
 (segment (start 127.05 75) (end 127.25 75.2) (width 0.4) (layer "F.Cu") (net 8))
 (segment (start 104.75 75) (end 127.05 75) (width 0.4) (layer "F.Cu") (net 8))
 (segment (start 129.75 75) (end 134 75) (width 0.5) (layer "F.Cu") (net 7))
 (segment (start 137 75) (end 137.2032 74.7968) (width 0.2) (layer "F.Cu") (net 7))
 (segment (start 137.2032 74.7968) (end 138.7 74.7968) (width 0.2) (layer "F.Cu") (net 7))
 (segment (start 134 75) (end 135 75) (width 0.3) (layer "F.Cu") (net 7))
 (via (at 137 75) (size 0.6) (drill 0.3) (layers "F.Cu" "B.Cu") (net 7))
 (via (at 135 75) (size 0.6) (drill 0.3) (layers "F.Cu" "B.Cu") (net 7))
 (segment (start 135 75) (end 137 75) (width 0.3) (layer "B.Cu") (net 7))
 (segment (start 132 78.2) (end 131.85 78.35) (width 0.3) (layer "F.Cu") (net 3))
 (segment (start 135.4468 75.4032) (end 135.5968 75.4032) (width 0.3) (layer "F.Cu") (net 3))
 (segment (start 133.85 77) (end 135.4468 75.4032) (width 0.3) (layer "F.Cu") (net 3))
 (segment (start 42.7 76.1) (end 41.7865 75.1865) (width 0.3) (layer "F.Cu") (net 3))
 (segment (start 44.05 78.35) (end 42.7 77) (width 0.3) (layer "F.Cu") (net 3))
 (segment (start 41.8032 75.2032) (end 42.5 75.9) (width 0.2) (layer "F.Cu") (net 3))
 (segment (start 131.85 78.35) (end 44.05 78.35) (width 0.3) (layer "F.Cu") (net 3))
 (segment (start 135.7968 75.2032) (end 136.3 75.2032) (width 0.2) (layer "F.Cu") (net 3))
 (segment (start 42.7 77) (end 42.7 76.1) (width 0.3) (layer "F.Cu") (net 3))
 (segment (start 132.5 77) (end 133.85 77) (width 0.3) (layer "F.Cu") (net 3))
 (segment (start 41.3 75.2032) (end 41.8032 75.2032) (width 0.2) (layer "F.Cu") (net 3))
 (segment (start 135.5968 75.4032) (end 135.7968 75.2032) (width 0.2) (layer "F.Cu") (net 3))
 (segment (start 41.7865 75.1865) (end 42.5 75.9) (width 0.3) (layer "F.Cu") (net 3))
 (via (at 132.5 77) (size 0.6) (drill 0.3) (layers "F.Cu" "B.Cu") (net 3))
 (via (at 132 78.2) (size 0.6) (drill 0.3) (layers "F.Cu" "B.Cu") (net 3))
 (segment (start 132.5 77) (end 132 77.5) (width 0.3) (layer "B.Cu") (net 3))
 (segment (start 132 77.5) (end 132 78.2) (width 0.3) (layer "B.Cu") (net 3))
 (segment (start 43.7 75.2032) (end 44.1968 75.2032) (width 0.2) (layer "F.Cu") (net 6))
 (segment (start 44.2 75.2) (end 44.4 75.4) (width 0.2) (layer "F.Cu") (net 6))
 (segment (start 138.3634 75.2032) (end 138.2968 75.2032) (width 0.3) (layer "F.Cu") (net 6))
 (segment (start 137.6 77) (end 137 77.6) (width 0.3) (layer "F.Cu") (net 6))
 (segment (start 44.85 77.6) (end 44.4 77.15) (width 0.3) (layer "F.Cu") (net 6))
 (segment (start 44.4 77.15) (end 44.4 75.4) (width 0.3) (layer "F.Cu") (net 6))
 (segment (start 138.3634 75.2032) (end 138.7 75.2032) (width 0.2) (layer "F.Cu") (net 6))
 (segment (start 138.2968 75.2032) (end 137.6 75.9) (width 0.3) (layer "F.Cu") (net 6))
 (segment (start 137.6 75.9) (end 137.6 77) (width 0.3) (layer "F.Cu") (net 6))
 (segment (start 137 77.6) (end 44.85 77.6) (width 0.3) (layer "F.Cu") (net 6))
 (segment (start 44.1968 75.2032) (end 44.2 75.2) (width 0.2) (layer "F.Cu") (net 6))
 (segment (start 41.9032 74.7968) (end 41.3 74.7968) (width 0.2) (layer "F.Cu") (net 2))
 (segment (start 42.4 74) (end 44.6 71.8) (width 0.3) (layer "F.Cu") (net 2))
 (segment (start 135.737096 74.7968) (end 135.370148 74.429852) (width 0.2) (layer "F.Cu") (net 2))
 (segment (start 132.6 72.2) (end 133.140296 72.2) (width 0.3) (layer "F.Cu") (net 2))
 (segment (start 132.2 71.8) (end 132.6 72.2) (width 0.3) (layer "F.Cu") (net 2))
 (segment (start 42.4 74.3) (end 41.9032 74.7968) (width 0.2) (layer "F.Cu") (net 2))
 (segment (start 136.3 74.7968) (end 135.737096 74.7968) (width 0.2) (layer "F.Cu") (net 2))
 (segment (start 133.140296 72.2) (end 135.370148 74.429852) (width 0.3) (layer "F.Cu") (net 2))
 (segment (start 42.4 74.3) (end 42.4 74) (width 0.3) (layer "F.Cu") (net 2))
 (segment (start 44.6 71.8) (end 132.2 71.8) (width 0.3) (layer "F.Cu") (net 2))
 (segment (start 47.2 75) (end 52.25 75) (width 0.3) (layer "F.Cu") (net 11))
 (segment (start 47 74.8) (end 47.2 75) (width 0.3) (layer "F.Cu") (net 11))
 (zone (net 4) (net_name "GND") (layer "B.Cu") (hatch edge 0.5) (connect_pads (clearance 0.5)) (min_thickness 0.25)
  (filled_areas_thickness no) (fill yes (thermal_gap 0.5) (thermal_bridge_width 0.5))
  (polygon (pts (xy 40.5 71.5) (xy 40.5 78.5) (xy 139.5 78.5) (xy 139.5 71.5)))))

